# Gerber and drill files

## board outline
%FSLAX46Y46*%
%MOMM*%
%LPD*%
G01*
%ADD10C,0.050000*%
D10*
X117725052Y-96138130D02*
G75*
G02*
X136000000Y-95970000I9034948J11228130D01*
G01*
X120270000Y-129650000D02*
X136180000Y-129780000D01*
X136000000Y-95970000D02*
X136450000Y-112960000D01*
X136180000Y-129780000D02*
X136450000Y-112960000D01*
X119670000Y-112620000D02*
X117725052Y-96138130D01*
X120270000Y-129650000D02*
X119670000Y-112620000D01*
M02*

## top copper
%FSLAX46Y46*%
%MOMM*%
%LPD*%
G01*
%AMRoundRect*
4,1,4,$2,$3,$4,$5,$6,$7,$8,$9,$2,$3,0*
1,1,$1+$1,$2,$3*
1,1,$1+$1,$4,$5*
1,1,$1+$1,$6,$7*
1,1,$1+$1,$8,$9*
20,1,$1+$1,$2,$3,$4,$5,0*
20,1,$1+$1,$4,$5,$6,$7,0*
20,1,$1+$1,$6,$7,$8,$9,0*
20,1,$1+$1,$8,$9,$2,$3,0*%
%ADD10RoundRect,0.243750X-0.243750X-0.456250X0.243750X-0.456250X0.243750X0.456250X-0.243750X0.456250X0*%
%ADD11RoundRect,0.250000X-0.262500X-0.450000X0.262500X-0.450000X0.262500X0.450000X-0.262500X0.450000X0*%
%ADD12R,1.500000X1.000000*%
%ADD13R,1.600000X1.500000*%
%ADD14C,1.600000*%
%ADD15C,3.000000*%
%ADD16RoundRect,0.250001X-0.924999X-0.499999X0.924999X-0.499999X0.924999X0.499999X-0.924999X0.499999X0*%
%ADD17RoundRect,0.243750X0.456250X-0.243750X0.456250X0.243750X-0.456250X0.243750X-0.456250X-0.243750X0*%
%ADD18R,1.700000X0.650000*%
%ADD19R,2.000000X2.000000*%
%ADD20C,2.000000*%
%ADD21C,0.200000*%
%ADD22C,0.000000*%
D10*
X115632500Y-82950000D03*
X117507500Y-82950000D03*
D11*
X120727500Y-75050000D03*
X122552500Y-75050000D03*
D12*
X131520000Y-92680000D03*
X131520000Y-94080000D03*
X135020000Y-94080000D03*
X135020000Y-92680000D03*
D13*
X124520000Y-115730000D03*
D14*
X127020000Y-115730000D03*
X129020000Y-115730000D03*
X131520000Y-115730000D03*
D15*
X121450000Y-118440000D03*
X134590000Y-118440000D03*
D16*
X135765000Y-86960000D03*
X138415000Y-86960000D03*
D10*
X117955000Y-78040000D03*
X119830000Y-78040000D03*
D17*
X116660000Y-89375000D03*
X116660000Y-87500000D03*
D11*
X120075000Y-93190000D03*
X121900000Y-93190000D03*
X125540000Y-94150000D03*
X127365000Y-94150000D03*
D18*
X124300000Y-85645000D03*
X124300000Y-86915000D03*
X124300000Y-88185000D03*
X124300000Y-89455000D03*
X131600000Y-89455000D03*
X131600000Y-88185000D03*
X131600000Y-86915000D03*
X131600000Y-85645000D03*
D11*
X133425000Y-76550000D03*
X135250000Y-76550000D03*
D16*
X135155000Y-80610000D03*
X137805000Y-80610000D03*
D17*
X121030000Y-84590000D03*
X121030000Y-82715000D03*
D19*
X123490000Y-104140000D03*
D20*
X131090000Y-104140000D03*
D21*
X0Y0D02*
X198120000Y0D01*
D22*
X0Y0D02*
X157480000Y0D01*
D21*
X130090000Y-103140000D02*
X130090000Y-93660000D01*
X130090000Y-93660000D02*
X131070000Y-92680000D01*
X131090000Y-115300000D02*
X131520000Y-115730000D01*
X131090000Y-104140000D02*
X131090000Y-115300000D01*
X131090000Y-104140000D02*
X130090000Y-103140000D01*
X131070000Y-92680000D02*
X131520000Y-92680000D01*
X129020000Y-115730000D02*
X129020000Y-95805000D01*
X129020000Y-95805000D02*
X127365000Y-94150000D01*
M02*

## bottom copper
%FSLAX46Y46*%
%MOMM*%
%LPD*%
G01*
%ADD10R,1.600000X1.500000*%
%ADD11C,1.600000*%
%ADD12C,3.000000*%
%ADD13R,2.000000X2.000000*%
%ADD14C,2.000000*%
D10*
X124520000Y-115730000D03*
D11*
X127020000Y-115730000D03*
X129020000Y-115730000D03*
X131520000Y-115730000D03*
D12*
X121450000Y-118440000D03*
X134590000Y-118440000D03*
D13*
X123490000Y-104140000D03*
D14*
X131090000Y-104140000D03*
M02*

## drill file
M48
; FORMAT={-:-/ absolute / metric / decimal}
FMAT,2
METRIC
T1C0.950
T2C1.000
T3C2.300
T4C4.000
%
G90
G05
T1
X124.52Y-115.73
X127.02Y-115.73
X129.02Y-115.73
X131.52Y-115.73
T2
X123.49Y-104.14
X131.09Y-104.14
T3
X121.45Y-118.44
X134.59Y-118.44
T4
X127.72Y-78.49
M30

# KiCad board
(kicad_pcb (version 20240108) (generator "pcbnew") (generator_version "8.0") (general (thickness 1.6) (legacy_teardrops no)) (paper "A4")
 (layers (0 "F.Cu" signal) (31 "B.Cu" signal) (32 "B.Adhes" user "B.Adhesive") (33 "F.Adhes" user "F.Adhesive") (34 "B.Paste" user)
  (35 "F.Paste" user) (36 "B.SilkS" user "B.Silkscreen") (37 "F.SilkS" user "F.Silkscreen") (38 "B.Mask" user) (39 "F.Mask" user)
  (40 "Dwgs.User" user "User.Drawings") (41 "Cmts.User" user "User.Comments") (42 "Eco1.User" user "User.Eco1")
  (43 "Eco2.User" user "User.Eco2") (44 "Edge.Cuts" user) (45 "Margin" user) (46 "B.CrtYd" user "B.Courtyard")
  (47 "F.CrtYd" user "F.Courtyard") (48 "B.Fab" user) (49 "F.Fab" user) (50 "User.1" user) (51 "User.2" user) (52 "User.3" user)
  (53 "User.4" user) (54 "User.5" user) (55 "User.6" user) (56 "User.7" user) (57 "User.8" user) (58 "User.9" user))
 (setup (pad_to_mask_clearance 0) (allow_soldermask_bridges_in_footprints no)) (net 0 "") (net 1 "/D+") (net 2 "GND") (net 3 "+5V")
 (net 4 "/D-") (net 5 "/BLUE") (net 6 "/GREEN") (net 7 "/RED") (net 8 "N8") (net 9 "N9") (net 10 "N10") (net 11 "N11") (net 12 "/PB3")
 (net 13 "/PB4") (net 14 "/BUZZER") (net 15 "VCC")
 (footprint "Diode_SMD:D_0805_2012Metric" (layer "F.Cu") (at 116.57 82.95)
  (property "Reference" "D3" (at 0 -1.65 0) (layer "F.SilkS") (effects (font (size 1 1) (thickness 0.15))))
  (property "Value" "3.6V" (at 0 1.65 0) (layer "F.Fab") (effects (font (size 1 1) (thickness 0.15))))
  (pad "1" smd roundrect (at -0.9375 0) (size 0.975 1.4) (layers "F.Cu" "F.Paste" "F.Mask") (roundrect_rratio 0.25) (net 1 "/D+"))
  (pad "2" smd roundrect (at 0.9375 0) (size 0.975 1.4) (layers "F.Cu" "F.Paste" "F.Mask") (roundrect_rratio 0.25) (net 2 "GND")))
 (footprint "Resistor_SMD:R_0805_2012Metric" (layer "F.Cu") (at 121.64 75.05)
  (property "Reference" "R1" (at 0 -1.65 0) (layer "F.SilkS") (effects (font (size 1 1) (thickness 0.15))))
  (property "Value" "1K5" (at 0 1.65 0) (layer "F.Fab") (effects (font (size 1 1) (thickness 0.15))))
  (pad "1" smd roundrect (at -0.9125 0) (size 1.025 1.4) (layers "F.Cu" "F.Paste" "F.Mask") (roundrect_rratio 0.243902) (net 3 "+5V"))
  (pad "2" smd roundrect (at 0.9125 0) (size 1.025 1.4) (layers "F.Cu" "F.Paste" "F.Mask") (roundrect_rratio 0.243902) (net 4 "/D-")))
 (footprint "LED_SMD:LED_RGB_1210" (layer "F.Cu") (at 133.27 93.38)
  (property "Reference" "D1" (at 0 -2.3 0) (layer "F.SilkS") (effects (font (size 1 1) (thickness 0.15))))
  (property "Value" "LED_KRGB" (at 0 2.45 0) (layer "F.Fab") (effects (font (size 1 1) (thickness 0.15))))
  (pad "1" smd rect (at -1.75 -0.7 180) (size 1.5 1) (layers "F.Cu" "F.Paste" "F.Mask") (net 2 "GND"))
  (pad "2" smd rect (at -1.75 0.7 180) (size 1.5 1) (layers "F.Cu" "F.Paste" "F.Mask") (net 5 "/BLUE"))
  (pad "3" smd rect (at 1.75 0.7 180) (size 1.5 1) (layers "F.Cu" "F.Paste" "F.Mask") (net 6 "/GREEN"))
  (pad "4" smd rect (at 1.75 -0.7 180) (size 1.5 1) (layers "F.Cu" "F.Paste" "F.Mask") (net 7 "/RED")))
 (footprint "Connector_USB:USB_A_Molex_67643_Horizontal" (layer "F.Cu") (at 124.52 115.73)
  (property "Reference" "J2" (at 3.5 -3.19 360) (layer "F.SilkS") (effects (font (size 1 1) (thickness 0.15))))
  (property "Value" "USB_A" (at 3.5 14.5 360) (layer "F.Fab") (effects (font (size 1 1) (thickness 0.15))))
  (pad "1" thru_hole rect (at 0 0) (size 1.6 1.5) (drill 0.95) (layers "*.Cu" "*.Mask") (remove_unused_layers no) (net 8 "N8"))
  (pad "2" thru_hole circle (at 2.5 0) (size 1.6 1.6) (drill 0.95) (layers "*.Cu" "*.Mask") (remove_unused_layers no) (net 4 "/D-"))
  (pad "3" thru_hole circle (at 4.5 0) (size 1.6 1.6) (drill 0.95) (layers "*.Cu" "*.Mask") (remove_unused_layers no) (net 1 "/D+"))
  (pad "4" thru_hole circle (at 7 0) (size 1.6 1.6) (drill 0.95) (layers "*.Cu" "*.Mask") (remove_unused_layers no) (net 2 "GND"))
  (pad "5" thru_hole circle (at -3.07 2.71) (size 3 3) (drill 2.3) (layers "*.Cu" "*.Mask") (remove_unused_layers no) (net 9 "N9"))
  (pad "5" thru_hole circle (at 10.07 2.71) (size 3 3) (drill 2.3) (layers "*.Cu" "*.Mask") (remove_unused_layers no) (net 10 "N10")))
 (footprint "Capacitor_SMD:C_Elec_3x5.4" (layer "F.Cu") (at 137.09 86.96)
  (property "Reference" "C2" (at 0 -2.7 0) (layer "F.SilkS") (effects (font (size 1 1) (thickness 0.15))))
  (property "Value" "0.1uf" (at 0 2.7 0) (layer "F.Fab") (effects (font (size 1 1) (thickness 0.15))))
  (pad "1" smd roundrect (at -1.325 0) (size 2.35 1.5) (layers "F.Cu" "F.Paste" "F.Mask") (roundrect_rratio 0.166667) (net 3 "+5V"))
  (pad "2" smd roundrect (at 1.325 0) (size 2.35 1.5) (layers "F.Cu" "F.Paste" "F.Mask") (roundrect_rratio 0.166667) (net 2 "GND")))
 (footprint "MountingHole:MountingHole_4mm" (layer "F.Cu") (at 127.72 78.49)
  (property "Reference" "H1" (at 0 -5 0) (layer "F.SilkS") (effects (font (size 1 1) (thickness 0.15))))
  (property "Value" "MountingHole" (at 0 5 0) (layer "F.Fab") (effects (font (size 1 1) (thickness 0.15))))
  (pad "" np_thru_hole circle (at 0 0) (size 4 4) (drill 4) (layers "*.Cu" "*.Mask")))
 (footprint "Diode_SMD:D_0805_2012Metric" (layer "F.Cu") (at 118.8925 78.04)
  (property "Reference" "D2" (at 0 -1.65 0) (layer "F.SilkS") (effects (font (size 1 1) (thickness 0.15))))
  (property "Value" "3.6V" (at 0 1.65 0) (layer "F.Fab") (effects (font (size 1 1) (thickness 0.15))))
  (pad "1" smd roundrect (at -0.9375 0) (size 0.975 1.4) (layers "F.Cu" "F.Paste" "F.Mask") (roundrect_rratio 0.25) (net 4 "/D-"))
  (pad "2" smd roundrect (at 0.9375 0) (size 0.975 1.4) (layers "F.Cu" "F.Paste" "F.Mask") (roundrect_rratio 0.25) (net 2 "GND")))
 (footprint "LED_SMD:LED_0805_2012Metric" (layer "F.Cu") (at 116.66 88.4375 90)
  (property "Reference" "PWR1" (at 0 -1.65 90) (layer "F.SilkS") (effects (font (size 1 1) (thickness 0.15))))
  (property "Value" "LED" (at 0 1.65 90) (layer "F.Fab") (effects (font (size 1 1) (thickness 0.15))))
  (pad "1" smd roundrect (at -0.9375 0 90) (size 0.975 1.4) (layers "F.Cu" "F.Paste" "F.Mask") (roundrect_rratio 0.25) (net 3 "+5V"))
  (pad "2" smd roundrect (at 0.9375 0 90) (size 0.975 1.4) (layers "F.Cu" "F.Paste" "F.Mask") (roundrect_rratio 0.25) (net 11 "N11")))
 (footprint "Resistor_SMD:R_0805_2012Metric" (layer "F.Cu") (at 120.9875 93.19)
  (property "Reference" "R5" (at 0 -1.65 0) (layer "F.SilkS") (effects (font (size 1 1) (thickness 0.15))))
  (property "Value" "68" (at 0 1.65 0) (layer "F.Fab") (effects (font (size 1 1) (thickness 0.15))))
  (pad "1" smd roundrect (at -0.9125 0) (size 1.025 1.4) (layers "F.Cu" "F.Paste" "F.Mask") (roundrect_rratio 0.243902) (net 4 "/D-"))
  (pad "2" smd roundrect (at 0.9125 0) (size 1.025 1.4) (layers "F.Cu" "F.Paste" "F.Mask") (roundrect_rratio 0.243902) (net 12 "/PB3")))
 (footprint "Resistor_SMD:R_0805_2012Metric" (layer "F.Cu") (at 126.4525 94.15)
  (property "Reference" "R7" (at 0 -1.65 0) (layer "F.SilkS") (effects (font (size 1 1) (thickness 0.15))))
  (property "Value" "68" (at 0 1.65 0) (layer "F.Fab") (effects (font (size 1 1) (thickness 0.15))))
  (pad "1" smd roundrect (at -0.9125 0) (size 1.025 1.4) (layers "F.Cu" "F.Paste" "F.Mask") (roundrect_rratio 0.243902) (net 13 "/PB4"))
  (pad "2" smd roundrect (at 0.9125 0) (size 1.025 1.4) (layers "F.Cu" "F.Paste" "F.Mask") (roundrect_rratio 0.243902) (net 1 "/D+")))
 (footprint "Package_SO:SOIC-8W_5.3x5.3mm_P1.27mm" (layer "F.Cu") (at 127.95 87.55)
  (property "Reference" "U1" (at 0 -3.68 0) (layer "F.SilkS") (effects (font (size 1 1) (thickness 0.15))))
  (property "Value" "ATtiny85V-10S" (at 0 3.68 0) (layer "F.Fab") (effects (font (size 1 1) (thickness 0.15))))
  (pad "1" smd rect (at -3.65 -1.905) (size 1.7 0.65) (layers "F.Cu" "F.Paste" "F.Mask") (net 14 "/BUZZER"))
  (pad "2" smd rect (at -3.65 -0.635) (size 1.7 0.65) (layers "F.Cu" "F.Paste" "F.Mask") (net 13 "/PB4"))
  (pad "3" smd rect (at -3.65 0.635) (size 1.7 0.65) (layers "F.Cu" "F.Paste" "F.Mask") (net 12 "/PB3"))
  (pad "4" smd rect (at -3.65 1.905) (size 1.7 0.65) (layers "F.Cu" "F.Paste" "F.Mask") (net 2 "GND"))
  (pad "5" smd rect (at 3.65 1.905) (size 1.7 0.65) (layers "F.Cu" "F.Paste" "F.Mask") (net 5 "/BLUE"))
  (pad "6" smd rect (at 3.65 0.635) (size 1.7 0.65) (layers "F.Cu" "F.Paste" "F.Mask") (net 6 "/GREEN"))
  (pad "7" smd rect (at 3.65 -0.635) (size 1.7 0.65) (layers "F.Cu" "F.Paste" "F.Mask") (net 7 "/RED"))
  (pad "8" smd rect (at 3.65 -1.905) (size 1.7 0.65) (layers "F.Cu" "F.Paste" "F.Mask") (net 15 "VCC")))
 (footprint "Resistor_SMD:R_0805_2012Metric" (layer "F.Cu") (at 134.3375 76.55)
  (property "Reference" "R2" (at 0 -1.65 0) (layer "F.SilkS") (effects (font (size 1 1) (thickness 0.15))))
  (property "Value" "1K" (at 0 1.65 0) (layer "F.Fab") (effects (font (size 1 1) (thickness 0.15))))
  (pad "1" smd roundrect (at -0.9125 0) (size 1.025 1.4) (layers "F.Cu" "F.Paste" "F.Mask") (roundrect_rratio 0.243902) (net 2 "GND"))
  (pad "2" smd roundrect (at 0.9125 0) (size 1.025 1.4) (layers "F.Cu" "F.Paste" "F.Mask") (roundrect_rratio 0.243902) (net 11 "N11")))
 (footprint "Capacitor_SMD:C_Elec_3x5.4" (layer "F.Cu") (at 136.48 80.61)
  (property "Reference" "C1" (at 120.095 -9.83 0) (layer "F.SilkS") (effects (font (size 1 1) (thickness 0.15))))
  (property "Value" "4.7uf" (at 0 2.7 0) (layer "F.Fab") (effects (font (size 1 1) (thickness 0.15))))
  (pad "1" smd roundrect (at -1.325 0) (size 2.35 1.5) (layers "F.Cu" "F.Paste" "F.Mask") (roundrect_rratio 0.166667) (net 3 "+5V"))
  (pad "2" smd roundrect (at 1.325 0) (size 2.35 1.5) (layers "F.Cu" "F.Paste" "F.Mask") (roundrect_rratio 0.166667) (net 2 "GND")))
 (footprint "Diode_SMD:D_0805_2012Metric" (layer "F.Cu") (at 121.03 83.6525 90)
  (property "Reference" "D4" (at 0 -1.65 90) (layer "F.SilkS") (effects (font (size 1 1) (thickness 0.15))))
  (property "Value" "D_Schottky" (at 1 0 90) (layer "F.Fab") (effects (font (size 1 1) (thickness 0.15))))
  (pad "1" smd roundrect (at -0.9375 0 90) (size 0.975 1.4) (layers "F.Cu" "F.Paste" "F.Mask") (roundrect_rratio 0.25) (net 8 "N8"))
  (pad "2" smd roundrect (at 0.9375 0 90) (size 0.975 1.4) (layers "F.Cu" "F.Paste" "F.Mask") (roundrect_rratio 0.25) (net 3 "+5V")))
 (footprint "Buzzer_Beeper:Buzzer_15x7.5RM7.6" (layer "F.Cu") (at 123.49 104.14)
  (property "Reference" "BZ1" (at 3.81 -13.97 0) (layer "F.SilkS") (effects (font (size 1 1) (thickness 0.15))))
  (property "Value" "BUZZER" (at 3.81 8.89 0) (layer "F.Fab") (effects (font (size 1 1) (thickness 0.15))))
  (pad "1" thru_hole rect (at 0 0) (size 2 2) (drill 1) (layers "*.Cu" "*.Mask") (remove_unused_layers no) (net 14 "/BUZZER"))
  (pad "2" thru_hole circle (at 7.6 0) (size 2 2) (drill 1) (layers "*.Cu" "*.Mask") (remove_unused_layers no) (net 2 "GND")))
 (gr_arc (start 117.725052 96.13813) (mid 126.627416 70.498768) (end 136 95.97) (stroke (width 0.05) (type default)) (layer "Edge.Cuts"))
 (gr_line (start 120.27 129.65) (end 136.18 129.78) (stroke (width 0.05) (type default)) (layer "Edge.Cuts"))
 (gr_line (start 136 95.97) (end 136.45 112.96) (stroke (width 0.05) (type default)) (layer "Edge.Cuts"))
 (gr_line (start 136.18 129.78) (end 136.45 112.96) (stroke (width 0.05) (type default)) (layer "Edge.Cuts"))
 (gr_line (start 119.67 112.62) (end 117.725052 96.13813) (stroke (width 0.05) (type default)) (layer "Edge.Cuts"))
 (gr_line (start 120.27 129.65) (end 119.67 112.62) (stroke (width 0.05) (type default)) (layer "Edge.Cuts"))
 (segment (start 0 0) (end 198.12 0) (width 0.2) (layer "F.Cu") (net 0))
 (segment (start 0 0) (end 157.48 0) (width 0) (layer "F.Cu") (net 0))
 (segment (start 130.09 103.14) (end 130.09 93.66) (width 0.2) (layer "F.Cu") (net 2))
 (segment (start 130.09 93.66) (end 131.07 92.68) (width 0.2) (layer "F.Cu") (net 2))
 (segment (start 131.09 115.3) (end 131.52 115.73) (width 0.2) (layer "F.Cu") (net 2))
 (segment (start 131.09 104.14) (end 131.09 115.3) (width 0.2) (layer "F.Cu") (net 2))
 (segment (start 131.09 104.14) (end 130.09 103.14) (width 0.2) (layer "F.Cu") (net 2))
 (segment (start 131.07 92.68) (end 131.52 92.68) (width 0.2) (layer "F.Cu") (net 2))
 (segment (start 129.02 115.73) (end 129.02 95.805) (width 0.2) (layer "F.Cu") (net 1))
 (segment (start 129.02 95.805) (end 127.365 94.15) (width 0.2) (layer "F.Cu") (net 1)))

